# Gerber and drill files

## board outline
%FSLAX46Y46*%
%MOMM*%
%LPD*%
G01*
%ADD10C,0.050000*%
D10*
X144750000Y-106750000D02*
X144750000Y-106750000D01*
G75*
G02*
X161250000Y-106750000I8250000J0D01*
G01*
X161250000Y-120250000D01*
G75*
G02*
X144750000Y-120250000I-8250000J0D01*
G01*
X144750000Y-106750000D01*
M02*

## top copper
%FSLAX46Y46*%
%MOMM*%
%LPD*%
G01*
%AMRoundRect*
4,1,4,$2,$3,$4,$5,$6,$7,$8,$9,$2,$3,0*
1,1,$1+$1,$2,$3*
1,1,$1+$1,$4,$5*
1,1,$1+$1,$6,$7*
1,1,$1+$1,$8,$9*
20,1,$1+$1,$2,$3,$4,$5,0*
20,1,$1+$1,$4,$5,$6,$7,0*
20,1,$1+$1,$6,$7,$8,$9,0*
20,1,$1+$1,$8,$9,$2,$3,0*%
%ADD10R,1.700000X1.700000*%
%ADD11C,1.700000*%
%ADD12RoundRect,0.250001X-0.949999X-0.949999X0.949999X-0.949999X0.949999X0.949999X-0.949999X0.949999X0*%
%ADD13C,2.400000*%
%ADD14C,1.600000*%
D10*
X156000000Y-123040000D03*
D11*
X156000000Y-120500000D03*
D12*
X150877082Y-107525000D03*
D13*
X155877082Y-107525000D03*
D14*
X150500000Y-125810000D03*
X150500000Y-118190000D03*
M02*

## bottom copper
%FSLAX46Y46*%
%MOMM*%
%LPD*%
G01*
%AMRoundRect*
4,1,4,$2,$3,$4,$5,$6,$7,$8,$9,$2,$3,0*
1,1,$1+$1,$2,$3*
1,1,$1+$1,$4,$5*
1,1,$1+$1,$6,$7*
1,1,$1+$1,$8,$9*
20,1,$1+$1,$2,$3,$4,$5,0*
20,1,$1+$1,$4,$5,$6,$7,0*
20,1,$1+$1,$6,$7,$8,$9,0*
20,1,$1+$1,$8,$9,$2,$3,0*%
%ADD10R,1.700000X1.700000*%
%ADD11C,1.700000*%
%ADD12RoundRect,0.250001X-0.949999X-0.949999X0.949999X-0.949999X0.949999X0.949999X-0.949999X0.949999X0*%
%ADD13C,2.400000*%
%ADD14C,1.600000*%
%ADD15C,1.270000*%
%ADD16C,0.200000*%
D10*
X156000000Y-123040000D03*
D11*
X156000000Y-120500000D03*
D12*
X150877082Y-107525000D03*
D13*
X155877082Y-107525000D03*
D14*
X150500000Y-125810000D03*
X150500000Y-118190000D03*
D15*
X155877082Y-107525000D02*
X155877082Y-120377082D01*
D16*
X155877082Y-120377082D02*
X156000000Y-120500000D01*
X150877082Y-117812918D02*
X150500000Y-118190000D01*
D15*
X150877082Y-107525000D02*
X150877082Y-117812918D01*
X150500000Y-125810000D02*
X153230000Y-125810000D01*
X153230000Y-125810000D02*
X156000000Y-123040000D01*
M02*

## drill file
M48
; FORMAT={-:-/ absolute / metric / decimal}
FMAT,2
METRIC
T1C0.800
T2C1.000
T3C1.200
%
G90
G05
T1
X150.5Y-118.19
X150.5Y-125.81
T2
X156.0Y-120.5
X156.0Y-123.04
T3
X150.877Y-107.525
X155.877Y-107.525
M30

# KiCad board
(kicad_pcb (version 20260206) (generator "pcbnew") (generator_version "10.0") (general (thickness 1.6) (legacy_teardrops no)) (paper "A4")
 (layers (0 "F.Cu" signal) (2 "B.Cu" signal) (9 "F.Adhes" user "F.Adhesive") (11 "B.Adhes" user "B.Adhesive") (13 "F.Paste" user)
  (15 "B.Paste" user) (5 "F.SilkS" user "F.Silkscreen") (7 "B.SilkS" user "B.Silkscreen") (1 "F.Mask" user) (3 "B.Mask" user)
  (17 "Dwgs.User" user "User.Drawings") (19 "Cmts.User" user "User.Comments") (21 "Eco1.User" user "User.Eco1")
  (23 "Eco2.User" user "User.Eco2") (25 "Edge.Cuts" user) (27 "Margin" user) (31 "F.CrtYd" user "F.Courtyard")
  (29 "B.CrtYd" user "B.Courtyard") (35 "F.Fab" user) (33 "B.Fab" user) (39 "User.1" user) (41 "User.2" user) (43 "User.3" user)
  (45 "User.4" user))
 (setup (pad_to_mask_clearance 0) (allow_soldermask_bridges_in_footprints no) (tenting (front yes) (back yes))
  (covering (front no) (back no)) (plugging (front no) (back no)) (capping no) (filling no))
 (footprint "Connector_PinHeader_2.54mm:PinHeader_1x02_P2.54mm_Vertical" (layer "F.Cu") (at 156 123.04 180)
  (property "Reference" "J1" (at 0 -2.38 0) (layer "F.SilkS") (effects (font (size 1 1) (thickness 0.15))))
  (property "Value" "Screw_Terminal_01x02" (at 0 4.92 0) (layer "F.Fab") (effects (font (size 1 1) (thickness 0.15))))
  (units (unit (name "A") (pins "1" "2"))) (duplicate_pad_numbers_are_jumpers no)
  (pad "1" thru_hole rect (at 0 0 180) (size 1.7 1.7) (drill 1) (layers "*.Cu" "*.Mask") (remove_unused_layers no) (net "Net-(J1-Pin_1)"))
  (pad "2" thru_hole circle (at 0 2.54 180) (size 1.7 1.7) (drill 1) (layers "*.Cu" "*.Mask") (remove_unused_layers no) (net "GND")))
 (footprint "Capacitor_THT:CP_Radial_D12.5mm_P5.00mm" (layer "F.Cu") (at 150.877082 107.525)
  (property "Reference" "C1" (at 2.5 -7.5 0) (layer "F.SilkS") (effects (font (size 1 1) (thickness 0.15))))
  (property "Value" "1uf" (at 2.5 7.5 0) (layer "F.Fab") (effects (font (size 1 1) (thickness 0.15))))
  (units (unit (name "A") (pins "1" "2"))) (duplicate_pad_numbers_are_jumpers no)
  (pad "1" thru_hole roundrect (at 0 0) (size 2.4 2.4) (drill 1.2) (layers "*.Cu" "*.Mask") (remove_unused_layers no)
   (roundrect_rratio 0.104167) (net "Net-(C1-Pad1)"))
  (pad "2" thru_hole circle (at 5 0) (size 2.4 2.4) (drill 1.2) (layers "*.Cu" "*.Mask") (remove_unused_layers no) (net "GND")))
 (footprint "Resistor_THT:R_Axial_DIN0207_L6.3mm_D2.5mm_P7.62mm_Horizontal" (layer "F.Cu") (at 150.5 125.81 90)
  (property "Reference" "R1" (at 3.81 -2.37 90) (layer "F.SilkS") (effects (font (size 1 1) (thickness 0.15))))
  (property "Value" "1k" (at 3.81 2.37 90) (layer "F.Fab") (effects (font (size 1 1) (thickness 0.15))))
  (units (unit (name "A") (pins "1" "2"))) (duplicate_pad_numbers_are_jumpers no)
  (pad "1" thru_hole circle (at 0 0 90) (size 1.6 1.6) (drill 0.8) (layers "*.Cu" "*.Mask") (remove_unused_layers no) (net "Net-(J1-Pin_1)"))
  (pad "2" thru_hole circle (at 7.62 0 90) (size 1.6 1.6) (drill 0.8) (layers "*.Cu" "*.Mask") (remove_unused_layers no)
   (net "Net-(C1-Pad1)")))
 (gr_rect (start 144.75 98.5) (end 161.25 128.5) (radius 8.25) (stroke (width 0.05) (type solid)) (fill no) (layer "Edge.Cuts"))
 (segment (start 155.877082 107.525) (end 155.877082 120.377082) (width 1.27) (layer "B.Cu") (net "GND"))
 (segment (start 155.877082 120.377082) (end 156 120.5) (width 0.2) (layer "B.Cu") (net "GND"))
 (segment (start 150.877082 117.812918) (end 150.5 118.19) (width 0.2) (layer "B.Cu") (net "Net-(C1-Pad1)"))
 (segment (start 150.877082 107.525) (end 150.877082 117.812918) (width 1.27) (layer "B.Cu") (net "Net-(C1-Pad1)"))
 (segment (start 150.5 125.81) (end 153.23 125.81) (width 1.27) (layer "B.Cu") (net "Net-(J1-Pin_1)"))
 (segment (start 153.23 125.81) (end 156 123.04) (width 1.27) (layer "B.Cu") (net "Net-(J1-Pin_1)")))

